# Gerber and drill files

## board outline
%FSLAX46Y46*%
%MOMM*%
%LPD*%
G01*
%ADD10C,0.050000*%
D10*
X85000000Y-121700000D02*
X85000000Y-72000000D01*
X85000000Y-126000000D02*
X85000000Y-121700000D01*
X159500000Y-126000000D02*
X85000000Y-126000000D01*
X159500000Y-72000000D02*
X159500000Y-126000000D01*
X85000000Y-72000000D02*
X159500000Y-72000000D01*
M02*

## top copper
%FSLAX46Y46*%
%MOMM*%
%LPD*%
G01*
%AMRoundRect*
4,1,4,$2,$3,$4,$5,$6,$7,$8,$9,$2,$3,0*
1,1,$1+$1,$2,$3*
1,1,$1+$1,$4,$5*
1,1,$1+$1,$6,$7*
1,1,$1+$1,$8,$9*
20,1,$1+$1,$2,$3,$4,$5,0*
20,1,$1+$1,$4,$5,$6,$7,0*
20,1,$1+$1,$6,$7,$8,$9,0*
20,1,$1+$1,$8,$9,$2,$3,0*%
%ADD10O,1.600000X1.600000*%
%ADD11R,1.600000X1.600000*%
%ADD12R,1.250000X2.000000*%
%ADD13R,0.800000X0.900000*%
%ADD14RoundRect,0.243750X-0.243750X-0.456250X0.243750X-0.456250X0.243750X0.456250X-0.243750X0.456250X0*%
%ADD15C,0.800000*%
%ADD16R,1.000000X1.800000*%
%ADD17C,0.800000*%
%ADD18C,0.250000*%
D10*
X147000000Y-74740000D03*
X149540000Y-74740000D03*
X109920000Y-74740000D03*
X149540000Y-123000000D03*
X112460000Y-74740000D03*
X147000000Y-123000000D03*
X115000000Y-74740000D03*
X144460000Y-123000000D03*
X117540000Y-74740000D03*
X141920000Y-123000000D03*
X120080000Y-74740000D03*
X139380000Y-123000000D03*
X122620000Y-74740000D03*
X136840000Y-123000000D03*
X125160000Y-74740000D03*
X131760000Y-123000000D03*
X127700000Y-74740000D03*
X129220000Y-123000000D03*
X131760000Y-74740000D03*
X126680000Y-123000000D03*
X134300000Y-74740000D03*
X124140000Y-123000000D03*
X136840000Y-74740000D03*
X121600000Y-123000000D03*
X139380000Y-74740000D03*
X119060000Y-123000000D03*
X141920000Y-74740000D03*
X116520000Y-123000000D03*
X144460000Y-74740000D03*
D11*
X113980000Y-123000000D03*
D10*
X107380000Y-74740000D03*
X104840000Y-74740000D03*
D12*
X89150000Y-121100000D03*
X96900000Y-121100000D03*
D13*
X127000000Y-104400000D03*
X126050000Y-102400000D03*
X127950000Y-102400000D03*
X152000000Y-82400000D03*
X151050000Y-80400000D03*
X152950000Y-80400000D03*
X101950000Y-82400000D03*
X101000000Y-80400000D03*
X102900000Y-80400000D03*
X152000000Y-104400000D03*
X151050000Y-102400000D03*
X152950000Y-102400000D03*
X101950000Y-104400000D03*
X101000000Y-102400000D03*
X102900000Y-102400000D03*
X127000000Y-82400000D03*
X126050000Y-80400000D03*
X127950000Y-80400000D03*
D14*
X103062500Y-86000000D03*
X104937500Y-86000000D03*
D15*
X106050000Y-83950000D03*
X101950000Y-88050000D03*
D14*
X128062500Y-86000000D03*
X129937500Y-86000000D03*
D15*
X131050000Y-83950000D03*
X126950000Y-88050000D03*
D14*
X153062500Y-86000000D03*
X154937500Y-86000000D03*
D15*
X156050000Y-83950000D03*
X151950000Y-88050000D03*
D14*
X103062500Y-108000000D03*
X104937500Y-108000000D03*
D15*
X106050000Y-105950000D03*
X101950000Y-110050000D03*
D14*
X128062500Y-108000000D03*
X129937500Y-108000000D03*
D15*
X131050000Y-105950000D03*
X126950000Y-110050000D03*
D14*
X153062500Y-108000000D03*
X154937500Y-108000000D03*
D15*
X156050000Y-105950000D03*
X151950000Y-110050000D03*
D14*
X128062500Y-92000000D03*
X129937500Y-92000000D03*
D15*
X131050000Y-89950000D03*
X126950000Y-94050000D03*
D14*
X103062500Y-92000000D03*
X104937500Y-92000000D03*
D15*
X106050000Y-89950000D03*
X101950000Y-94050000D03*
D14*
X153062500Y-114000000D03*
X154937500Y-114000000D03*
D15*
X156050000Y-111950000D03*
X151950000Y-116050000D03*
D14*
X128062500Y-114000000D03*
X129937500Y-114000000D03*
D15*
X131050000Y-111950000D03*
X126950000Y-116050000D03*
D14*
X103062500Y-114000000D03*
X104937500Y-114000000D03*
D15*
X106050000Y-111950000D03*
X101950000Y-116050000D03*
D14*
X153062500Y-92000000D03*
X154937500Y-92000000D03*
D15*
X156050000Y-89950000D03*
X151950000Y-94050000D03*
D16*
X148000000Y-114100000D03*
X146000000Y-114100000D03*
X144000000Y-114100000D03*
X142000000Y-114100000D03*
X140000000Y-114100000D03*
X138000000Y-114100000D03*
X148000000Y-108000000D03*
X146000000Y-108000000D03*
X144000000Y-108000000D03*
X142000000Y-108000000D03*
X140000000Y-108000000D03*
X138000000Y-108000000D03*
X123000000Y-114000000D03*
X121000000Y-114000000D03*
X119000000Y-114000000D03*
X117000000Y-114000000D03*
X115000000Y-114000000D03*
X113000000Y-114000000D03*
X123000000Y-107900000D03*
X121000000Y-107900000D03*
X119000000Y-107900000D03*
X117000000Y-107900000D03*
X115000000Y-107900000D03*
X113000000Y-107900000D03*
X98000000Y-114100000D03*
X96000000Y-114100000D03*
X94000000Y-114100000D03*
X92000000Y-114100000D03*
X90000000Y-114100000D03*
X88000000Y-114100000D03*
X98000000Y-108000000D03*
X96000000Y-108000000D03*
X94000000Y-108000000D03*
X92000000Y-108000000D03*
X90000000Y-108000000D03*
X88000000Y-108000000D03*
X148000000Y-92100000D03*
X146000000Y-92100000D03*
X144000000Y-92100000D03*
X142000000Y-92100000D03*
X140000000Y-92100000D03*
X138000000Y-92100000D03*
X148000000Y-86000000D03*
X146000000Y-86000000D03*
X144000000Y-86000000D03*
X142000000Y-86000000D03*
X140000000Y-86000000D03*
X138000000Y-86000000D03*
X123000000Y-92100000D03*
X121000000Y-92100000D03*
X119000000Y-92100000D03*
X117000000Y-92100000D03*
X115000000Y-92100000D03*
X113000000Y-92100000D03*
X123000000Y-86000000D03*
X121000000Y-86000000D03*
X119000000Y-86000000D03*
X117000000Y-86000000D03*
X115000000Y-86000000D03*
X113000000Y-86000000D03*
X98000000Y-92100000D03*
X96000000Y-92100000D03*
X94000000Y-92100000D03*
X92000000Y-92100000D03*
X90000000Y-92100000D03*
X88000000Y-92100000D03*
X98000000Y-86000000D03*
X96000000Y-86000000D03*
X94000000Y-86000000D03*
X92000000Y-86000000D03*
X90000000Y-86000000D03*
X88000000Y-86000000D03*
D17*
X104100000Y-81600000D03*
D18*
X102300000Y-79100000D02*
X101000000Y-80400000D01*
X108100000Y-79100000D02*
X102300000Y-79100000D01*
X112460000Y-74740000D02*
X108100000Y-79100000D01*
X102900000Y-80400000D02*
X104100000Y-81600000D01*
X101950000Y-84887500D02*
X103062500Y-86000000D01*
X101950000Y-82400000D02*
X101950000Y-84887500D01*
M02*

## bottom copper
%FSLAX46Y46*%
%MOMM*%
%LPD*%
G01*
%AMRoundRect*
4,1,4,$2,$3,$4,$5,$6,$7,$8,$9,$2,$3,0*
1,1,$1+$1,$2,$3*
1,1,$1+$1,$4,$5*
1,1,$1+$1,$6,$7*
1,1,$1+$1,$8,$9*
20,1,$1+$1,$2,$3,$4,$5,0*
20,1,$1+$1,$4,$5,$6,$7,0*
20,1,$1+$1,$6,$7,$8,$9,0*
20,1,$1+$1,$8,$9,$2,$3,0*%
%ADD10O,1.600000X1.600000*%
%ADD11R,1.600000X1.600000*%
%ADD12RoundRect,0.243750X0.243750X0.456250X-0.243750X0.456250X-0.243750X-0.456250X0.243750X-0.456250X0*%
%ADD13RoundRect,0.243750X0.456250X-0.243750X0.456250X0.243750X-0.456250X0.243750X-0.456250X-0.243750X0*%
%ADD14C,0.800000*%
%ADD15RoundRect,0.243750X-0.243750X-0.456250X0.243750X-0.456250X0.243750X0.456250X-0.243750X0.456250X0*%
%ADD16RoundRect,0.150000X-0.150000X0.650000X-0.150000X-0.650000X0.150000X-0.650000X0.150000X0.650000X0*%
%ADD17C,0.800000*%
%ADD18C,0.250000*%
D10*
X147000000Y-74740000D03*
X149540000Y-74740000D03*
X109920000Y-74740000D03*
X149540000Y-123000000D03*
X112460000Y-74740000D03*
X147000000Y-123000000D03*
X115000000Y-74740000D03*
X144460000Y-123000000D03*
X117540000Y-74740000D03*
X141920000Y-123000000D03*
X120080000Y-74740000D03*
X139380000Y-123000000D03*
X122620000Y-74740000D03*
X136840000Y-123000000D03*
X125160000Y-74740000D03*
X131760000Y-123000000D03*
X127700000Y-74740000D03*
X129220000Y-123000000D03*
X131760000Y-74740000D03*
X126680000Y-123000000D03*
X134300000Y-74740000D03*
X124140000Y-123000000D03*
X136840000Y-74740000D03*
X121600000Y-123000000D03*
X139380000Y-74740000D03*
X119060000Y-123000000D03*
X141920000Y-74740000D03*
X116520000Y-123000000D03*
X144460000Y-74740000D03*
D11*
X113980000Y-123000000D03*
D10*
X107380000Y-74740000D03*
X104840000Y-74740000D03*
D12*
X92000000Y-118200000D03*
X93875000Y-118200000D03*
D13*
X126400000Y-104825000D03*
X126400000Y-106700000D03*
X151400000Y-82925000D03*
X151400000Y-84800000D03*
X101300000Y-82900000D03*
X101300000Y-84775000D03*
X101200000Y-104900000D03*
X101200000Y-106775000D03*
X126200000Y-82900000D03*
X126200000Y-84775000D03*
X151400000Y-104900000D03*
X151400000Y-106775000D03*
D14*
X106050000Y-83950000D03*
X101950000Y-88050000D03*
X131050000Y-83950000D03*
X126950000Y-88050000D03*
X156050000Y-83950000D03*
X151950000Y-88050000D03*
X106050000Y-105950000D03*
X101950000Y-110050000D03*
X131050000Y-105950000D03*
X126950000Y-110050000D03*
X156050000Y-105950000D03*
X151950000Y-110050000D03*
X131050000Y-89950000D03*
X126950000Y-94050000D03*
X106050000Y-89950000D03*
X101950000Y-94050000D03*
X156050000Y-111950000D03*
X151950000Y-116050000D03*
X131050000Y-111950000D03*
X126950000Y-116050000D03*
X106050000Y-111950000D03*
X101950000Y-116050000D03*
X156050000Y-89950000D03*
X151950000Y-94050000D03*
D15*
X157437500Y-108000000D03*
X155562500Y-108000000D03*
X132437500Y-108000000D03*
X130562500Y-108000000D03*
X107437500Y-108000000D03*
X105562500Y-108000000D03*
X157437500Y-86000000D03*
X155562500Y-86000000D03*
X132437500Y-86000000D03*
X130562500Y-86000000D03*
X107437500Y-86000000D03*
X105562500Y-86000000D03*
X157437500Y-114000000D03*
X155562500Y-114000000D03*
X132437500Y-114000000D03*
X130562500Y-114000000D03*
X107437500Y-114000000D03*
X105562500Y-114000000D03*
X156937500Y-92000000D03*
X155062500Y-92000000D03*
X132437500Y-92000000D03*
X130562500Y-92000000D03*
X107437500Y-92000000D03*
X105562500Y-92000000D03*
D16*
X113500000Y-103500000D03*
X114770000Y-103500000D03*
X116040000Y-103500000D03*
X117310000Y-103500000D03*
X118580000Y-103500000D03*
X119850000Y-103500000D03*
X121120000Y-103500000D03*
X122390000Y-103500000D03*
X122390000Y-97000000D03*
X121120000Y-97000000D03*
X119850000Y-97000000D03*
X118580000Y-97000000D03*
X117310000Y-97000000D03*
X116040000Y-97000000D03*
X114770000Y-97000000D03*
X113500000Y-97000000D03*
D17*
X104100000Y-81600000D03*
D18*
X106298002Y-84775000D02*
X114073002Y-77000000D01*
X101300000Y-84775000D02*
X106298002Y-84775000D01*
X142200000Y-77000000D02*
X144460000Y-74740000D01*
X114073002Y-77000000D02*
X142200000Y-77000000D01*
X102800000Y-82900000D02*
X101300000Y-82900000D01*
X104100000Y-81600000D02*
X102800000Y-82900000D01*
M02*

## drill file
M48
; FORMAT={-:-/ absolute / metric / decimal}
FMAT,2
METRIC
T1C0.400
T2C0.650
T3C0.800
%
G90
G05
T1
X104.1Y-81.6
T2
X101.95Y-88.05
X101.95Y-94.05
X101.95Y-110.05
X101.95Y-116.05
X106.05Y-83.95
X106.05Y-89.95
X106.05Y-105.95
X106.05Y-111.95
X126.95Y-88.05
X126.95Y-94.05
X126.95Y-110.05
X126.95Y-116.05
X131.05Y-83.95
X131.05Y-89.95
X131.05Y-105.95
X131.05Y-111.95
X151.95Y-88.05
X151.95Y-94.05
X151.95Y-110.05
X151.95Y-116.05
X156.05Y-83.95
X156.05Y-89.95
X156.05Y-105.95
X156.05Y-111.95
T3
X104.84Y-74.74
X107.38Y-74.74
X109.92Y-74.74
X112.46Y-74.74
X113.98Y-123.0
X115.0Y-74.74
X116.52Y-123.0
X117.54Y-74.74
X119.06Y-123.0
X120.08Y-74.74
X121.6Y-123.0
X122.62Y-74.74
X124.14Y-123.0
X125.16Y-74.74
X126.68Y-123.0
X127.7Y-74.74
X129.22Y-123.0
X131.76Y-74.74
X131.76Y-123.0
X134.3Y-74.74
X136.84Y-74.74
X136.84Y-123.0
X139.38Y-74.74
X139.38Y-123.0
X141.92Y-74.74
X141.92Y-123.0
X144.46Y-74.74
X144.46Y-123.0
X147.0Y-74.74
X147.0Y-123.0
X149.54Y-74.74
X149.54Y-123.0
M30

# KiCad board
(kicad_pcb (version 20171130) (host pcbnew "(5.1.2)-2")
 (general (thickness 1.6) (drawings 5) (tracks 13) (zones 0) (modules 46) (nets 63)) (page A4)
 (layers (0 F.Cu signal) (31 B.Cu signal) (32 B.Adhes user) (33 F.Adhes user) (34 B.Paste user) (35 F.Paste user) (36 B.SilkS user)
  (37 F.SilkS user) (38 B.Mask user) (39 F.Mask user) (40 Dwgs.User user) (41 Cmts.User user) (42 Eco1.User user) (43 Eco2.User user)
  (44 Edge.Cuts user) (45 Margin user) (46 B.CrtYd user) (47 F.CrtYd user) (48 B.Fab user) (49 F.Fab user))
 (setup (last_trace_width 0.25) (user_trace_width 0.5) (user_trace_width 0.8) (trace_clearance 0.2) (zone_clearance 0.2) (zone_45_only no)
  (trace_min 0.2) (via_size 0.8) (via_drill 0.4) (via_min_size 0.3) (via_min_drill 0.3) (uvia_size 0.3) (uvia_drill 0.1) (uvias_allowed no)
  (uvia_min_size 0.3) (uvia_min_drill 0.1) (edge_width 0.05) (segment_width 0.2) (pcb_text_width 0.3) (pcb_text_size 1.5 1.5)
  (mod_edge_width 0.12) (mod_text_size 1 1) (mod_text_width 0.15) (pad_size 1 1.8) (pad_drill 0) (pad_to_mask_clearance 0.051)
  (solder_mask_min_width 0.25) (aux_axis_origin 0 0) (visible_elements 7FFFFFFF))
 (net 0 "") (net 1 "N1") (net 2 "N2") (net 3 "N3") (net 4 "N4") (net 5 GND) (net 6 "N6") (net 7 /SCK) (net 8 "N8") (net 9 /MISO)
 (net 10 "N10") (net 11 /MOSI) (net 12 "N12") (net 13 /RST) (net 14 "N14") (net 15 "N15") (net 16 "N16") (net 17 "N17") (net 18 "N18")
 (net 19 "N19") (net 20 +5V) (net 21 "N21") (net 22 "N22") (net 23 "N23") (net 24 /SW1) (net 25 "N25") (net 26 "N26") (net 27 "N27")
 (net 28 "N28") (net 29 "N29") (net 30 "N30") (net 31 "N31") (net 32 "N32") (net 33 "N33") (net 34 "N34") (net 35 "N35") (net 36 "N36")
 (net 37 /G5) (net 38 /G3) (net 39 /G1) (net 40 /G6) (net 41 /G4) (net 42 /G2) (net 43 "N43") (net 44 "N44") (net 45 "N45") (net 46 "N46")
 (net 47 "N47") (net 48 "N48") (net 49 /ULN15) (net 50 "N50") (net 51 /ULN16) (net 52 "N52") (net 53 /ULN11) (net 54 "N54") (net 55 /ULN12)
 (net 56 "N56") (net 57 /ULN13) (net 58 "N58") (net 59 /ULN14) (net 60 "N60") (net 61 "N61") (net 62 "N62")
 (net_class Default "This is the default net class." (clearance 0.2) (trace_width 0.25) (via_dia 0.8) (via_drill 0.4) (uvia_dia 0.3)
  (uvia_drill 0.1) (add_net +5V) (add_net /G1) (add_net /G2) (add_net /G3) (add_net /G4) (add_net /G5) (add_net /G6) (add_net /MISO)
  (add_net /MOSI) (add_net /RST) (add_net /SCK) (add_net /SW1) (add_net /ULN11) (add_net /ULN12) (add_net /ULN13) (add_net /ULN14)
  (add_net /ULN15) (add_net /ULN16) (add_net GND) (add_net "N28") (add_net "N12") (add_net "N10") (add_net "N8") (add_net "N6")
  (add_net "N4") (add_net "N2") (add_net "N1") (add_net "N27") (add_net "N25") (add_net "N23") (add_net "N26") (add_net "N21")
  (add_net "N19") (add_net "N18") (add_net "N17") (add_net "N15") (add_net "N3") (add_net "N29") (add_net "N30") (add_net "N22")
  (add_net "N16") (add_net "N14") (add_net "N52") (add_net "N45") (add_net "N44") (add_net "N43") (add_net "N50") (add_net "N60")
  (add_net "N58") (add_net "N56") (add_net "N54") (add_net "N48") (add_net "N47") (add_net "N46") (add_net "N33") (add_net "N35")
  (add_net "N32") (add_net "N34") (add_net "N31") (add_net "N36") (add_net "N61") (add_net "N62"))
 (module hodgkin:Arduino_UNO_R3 (layer B.Cu) (at 113.98 123)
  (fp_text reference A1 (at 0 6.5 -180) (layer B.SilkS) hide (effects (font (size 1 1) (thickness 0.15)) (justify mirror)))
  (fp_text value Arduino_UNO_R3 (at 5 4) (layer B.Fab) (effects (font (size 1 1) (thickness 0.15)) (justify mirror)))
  (pad 16 thru_hole oval (at 33.02 -48.26 270) (size 1.6 1.6) (drill 0.8) (layers *.Cu *.Mask) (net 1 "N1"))
  (pad 15 thru_hole oval (at 35.56 -48.26 270) (size 1.6 1.6) (drill 0.8) (layers *.Cu *.Mask) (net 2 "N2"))
  (pad 30 thru_hole oval (at -4.06 -48.26 270) (size 1.6 1.6) (drill 0.8) (layers *.Cu *.Mask) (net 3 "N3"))
  (pad 14 thru_hole oval (at 35.56 0 270) (size 1.6 1.6) (drill 0.8) (layers *.Cu *.Mask) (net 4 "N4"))
  (pad 29 thru_hole oval (at -1.52 -48.26 270) (size 1.6 1.6) (drill 0.8) (layers *.Cu *.Mask) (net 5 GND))
  (pad 13 thru_hole oval (at 33.02 0 270) (size 1.6 1.6) (drill 0.8) (layers *.Cu *.Mask) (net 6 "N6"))
  (pad 28 thru_hole oval (at 1.02 -48.26 270) (size 1.6 1.6) (drill 0.8) (layers *.Cu *.Mask) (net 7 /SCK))
  (pad 12 thru_hole oval (at 30.48 0 270) (size 1.6 1.6) (drill 0.8) (layers *.Cu *.Mask) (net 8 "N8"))
  (pad 27 thru_hole oval (at 3.56 -48.26 270) (size 1.6 1.6) (drill 0.8) (layers *.Cu *.Mask) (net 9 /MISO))
  (pad 11 thru_hole oval (at 27.94 0 270) (size 1.6 1.6) (drill 0.8) (layers *.Cu *.Mask) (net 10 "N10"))
  (pad 26 thru_hole oval (at 6.1 -48.26 270) (size 1.6 1.6) (drill 0.8) (layers *.Cu *.Mask) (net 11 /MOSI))
  (pad 10 thru_hole oval (at 25.4 0 270) (size 1.6 1.6) (drill 0.8) (layers *.Cu *.Mask) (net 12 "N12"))
  (pad 25 thru_hole oval (at 8.64 -48.26 270) (size 1.6 1.6) (drill 0.8) (layers *.Cu *.Mask) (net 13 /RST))
  (pad 9 thru_hole oval (at 22.86 0 270) (size 1.6 1.6) (drill 0.8) (layers *.Cu *.Mask) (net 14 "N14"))
  (pad 24 thru_hole oval (at 11.18 -48.26 270) (size 1.6 1.6) (drill 0.8) (layers *.Cu *.Mask) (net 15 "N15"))
  (pad 8 thru_hole oval (at 17.78 0 270) (size 1.6 1.6) (drill 0.8) (layers *.Cu *.Mask) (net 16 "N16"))
  (pad 23 thru_hole oval (at 13.72 -48.26 270) (size 1.6 1.6) (drill 0.8) (layers *.Cu *.Mask) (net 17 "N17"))
  (pad 7 thru_hole oval (at 15.24 0 270) (size 1.6 1.6) (drill 0.8) (layers *.Cu *.Mask) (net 5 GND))
  (pad 22 thru_hole oval (at 17.78 -48.26 270) (size 1.6 1.6) (drill 0.8) (layers *.Cu *.Mask) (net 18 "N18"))
  (pad 6 thru_hole oval (at 12.7 0 270) (size 1.6 1.6) (drill 0.8) (layers *.Cu *.Mask) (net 5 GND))
  (pad 21 thru_hole oval (at 20.32 -48.26 270) (size 1.6 1.6) (drill 0.8) (layers *.Cu *.Mask) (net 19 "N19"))
  (pad 5 thru_hole oval (at 10.16 0 270) (size 1.6 1.6) (drill 0.8) (layers *.Cu *.Mask) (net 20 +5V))
  (pad 20 thru_hole oval (at 22.86 -48.26 270) (size 1.6 1.6) (drill 0.8) (layers *.Cu *.Mask) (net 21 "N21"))
  (pad 4 thru_hole oval (at 7.62 0 270) (size 1.6 1.6) (drill 0.8) (layers *.Cu *.Mask) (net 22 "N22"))
  (pad 19 thru_hole oval (at 25.4 -48.26 270) (size 1.6 1.6) (drill 0.8) (layers *.Cu *.Mask) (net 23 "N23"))
  (pad 3 thru_hole oval (at 5.08 0 270) (size 1.6 1.6) (drill 0.8) (layers *.Cu *.Mask) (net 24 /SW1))
  (pad 18 thru_hole oval (at 27.94 -48.26 270) (size 1.6 1.6) (drill 0.8) (layers *.Cu *.Mask) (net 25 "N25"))
  (pad 2 thru_hole oval (at 2.54 0 270) (size 1.6 1.6) (drill 0.8) (layers *.Cu *.Mask) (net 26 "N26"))
  (pad 17 thru_hole oval (at 30.48 -48.26 270) (size 1.6 1.6) (drill 0.8) (layers *.Cu *.Mask) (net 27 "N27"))
  (pad 1 thru_hole rect (at 0 0 270) (size 1.6 1.6) (drill 0.8) (layers *.Cu *.Mask) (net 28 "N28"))
  (pad 31 thru_hole oval (at -6.6 -48.26 270) (size 1.6 1.6) (drill 0.8) (layers *.Cu *.Mask) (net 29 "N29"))
  (pad 32 thru_hole oval (at -9.14 -48.26 270) (size 1.6 1.6) (drill 0.8) (layers *.Cu *.Mask) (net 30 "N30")))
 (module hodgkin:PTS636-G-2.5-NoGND (layer F.Cu) (at 96.9 121.1 180)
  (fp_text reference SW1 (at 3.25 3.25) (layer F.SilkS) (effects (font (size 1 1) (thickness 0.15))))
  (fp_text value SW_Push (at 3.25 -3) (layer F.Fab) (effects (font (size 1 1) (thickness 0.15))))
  (pad 2 smd rect (at 7.75 0 180) (size 1.25 2) (layers F.Cu F.Paste F.Mask) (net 24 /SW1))
  (pad 1 smd rect (at 0 0 180) (size 1.25 2) (layers F.Cu F.Paste F.Mask) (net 5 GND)))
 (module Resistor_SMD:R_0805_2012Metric (layer B.Cu) (at 92.9375 118.2 180)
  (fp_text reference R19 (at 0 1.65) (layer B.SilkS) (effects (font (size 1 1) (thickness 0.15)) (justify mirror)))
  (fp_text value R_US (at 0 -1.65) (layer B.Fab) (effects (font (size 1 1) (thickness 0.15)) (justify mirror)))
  (pad 2 smd roundrect (at 0.9375 0 180) (size 0.975 1.4) (layers B.Cu B.Paste B.Mask) (roundrect_rratio 0.25) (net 24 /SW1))
  (pad 1 smd roundrect (at -0.9375 0 180) (size 0.975 1.4) (layers B.Cu B.Paste B.Mask) (roundrect_rratio 0.25) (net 20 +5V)))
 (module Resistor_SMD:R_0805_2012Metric (layer B.Cu) (at 126.4 105.7625 90)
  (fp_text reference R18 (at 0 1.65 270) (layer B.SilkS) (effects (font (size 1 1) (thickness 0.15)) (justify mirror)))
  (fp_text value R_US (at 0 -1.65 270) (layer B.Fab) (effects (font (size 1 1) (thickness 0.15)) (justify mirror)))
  (pad 2 smd roundrect (at 0.9375 0 90) (size 0.975 1.4) (layers B.Cu B.Paste B.Mask) (roundrect_rratio 0.25) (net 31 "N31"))
  (pad 1 smd roundrect (at -0.9375 0 90) (size 0.975 1.4) (layers B.Cu B.Paste B.Mask) (roundrect_rratio 0.25) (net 6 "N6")))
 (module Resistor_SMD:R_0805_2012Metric (layer B.Cu) (at 151.4 83.8625 90)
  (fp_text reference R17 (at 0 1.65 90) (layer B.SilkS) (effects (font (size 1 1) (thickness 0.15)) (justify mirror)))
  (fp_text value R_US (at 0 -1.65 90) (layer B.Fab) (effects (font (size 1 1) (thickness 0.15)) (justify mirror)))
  (pad 2 smd roundrect (at 0.9375 0 90) (size 0.975 1.4) (layers B.Cu B.Paste B.Mask) (roundrect_rratio 0.25) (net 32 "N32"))
  (pad 1 smd roundrect (at -0.9375 0 90) (size 0.975 1.4) (layers B.Cu B.Paste B.Mask) (roundrect_rratio 0.25) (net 2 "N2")))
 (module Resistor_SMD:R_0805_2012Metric (layer B.Cu) (at 101.3 83.8375 90)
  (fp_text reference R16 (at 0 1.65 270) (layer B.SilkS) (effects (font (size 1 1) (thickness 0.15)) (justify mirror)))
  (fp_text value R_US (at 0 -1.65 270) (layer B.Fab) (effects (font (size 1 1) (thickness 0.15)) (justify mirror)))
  (pad 2 smd roundrect (at 0.9375 0 90) (size 0.975 1.4) (layers B.Cu B.Paste B.Mask) (roundrect_rratio 0.25) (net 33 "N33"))
  (pad 1 smd roundrect (at -0.9375 0 90) (size 0.975 1.4) (layers B.Cu B.Paste B.Mask) (roundrect_rratio 0.25) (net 27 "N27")))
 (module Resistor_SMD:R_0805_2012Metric (layer B.Cu) (at 101.2 105.8375 90)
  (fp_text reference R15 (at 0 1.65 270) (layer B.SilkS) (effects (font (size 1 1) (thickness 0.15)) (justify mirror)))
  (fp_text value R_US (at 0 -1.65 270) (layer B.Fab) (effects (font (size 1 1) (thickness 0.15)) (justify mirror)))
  (pad 2 smd roundrect (at 0.9375 0 90) (size 0.975 1.4) (layers B.Cu B.Paste B.Mask) (roundrect_rratio 0.25) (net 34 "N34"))
  (pad 1 smd roundrect (at -0.9375 0 90) (size 0.975 1.4) (layers B.Cu B.Paste B.Mask) (roundrect_rratio 0.25) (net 8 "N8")))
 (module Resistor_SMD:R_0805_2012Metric (layer B.Cu) (at 126.2 83.8375 90)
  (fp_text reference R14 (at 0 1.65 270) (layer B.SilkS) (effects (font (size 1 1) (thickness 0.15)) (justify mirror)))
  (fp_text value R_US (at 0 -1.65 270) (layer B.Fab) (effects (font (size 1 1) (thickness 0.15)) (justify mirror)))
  (pad 2 smd roundrect (at 0.9375 0 90) (size 0.975 1.4) (layers B.Cu B.Paste B.Mask) (roundrect_rratio 0.25) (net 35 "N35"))
  (pad 1 smd roundrect (at -0.9375 0 90) (size 0.975 1.4) (layers B.Cu B.Paste B.Mask) (roundrect_rratio 0.25) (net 1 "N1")))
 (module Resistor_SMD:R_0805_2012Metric (layer B.Cu) (at 151.4 105.8375 90)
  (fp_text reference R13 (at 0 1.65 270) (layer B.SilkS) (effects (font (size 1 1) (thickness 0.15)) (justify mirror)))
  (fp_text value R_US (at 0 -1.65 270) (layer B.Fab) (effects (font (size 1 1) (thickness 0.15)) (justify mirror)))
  (pad 2 smd roundrect (at 0.9375 0 90) (size 0.975 1.4) (layers B.Cu B.Paste B.Mask) (roundrect_rratio 0.25) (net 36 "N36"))
  (pad 1 smd roundrect (at -0.9375 0 90) (size 0.975 1.4) (layers B.Cu B.Paste B.Mask) (roundrect_rratio 0.25) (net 4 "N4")))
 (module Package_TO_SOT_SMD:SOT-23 (layer F.Cu) (at 127 103.4 270)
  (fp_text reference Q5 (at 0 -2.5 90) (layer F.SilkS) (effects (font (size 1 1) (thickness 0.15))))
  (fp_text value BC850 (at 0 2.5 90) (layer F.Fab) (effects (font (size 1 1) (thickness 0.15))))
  (pad 3 smd rect (at 1 0 270) (size 0.9 0.8) (layers F.Cu F.Paste F.Mask) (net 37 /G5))
  (pad 2 smd rect (at -1 0.95 270) (size 0.9 0.8) (layers F.Cu F.Paste F.Mask) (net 5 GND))
  (pad 1 smd rect (at -1 -0.95 270) (size 0.9 0.8) (layers F.Cu F.Paste F.Mask) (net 31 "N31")))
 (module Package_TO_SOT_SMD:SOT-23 (layer F.Cu) (at 152 81.4 270)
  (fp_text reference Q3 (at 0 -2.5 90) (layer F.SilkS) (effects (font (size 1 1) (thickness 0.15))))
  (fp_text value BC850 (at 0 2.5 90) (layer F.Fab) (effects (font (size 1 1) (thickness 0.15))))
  (pad 3 smd rect (at 1 0 270) (size 0.9 0.8) (layers F.Cu F.Paste F.Mask) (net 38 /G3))
  (pad 2 smd rect (at -1 0.95 270) (size 0.9 0.8) (layers F.Cu F.Paste F.Mask) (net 5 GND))
  (pad 1 smd rect (at -1 -0.95 270) (size 0.9 0.8) (layers F.Cu F.Paste F.Mask) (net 32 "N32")))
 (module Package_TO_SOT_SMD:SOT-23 (layer F.Cu) (at 101.95 81.4 270)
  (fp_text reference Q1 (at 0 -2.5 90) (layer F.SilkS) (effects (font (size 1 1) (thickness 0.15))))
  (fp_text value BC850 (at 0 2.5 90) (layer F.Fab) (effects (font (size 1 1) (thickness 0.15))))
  (pad 3 smd rect (at 1 0 270) (size 0.9 0.8) (layers F.Cu F.Paste F.Mask) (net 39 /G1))
  (pad 2 smd rect (at -1 0.95 270) (size 0.9 0.8) (layers F.Cu F.Paste F.Mask) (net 5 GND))
  (pad 1 smd rect (at -1 -0.95 270) (size 0.9 0.8) (layers F.Cu F.Paste F.Mask) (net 33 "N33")))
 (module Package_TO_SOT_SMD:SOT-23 (layer F.Cu) (at 152 103.4 270)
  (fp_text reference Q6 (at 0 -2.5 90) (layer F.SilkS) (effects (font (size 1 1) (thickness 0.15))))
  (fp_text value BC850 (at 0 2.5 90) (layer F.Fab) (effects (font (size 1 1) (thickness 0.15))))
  (pad 3 smd rect (at 1 0 270) (size 0.9 0.8) (layers F.Cu F.Paste F.Mask) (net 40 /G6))
  (pad 2 smd rect (at -1 0.95 270) (size 0.9 0.8) (layers F.Cu F.Paste F.Mask) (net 5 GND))
  (pad 1 smd rect (at -1 -0.95 270) (size 0.9 0.8) (layers F.Cu F.Paste F.Mask) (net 36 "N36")))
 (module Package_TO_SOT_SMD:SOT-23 (layer F.Cu) (at 101.95 103.4 270)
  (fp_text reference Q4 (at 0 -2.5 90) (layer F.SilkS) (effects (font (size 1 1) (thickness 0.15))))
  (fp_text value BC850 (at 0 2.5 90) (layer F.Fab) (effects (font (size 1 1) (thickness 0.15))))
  (pad 3 smd rect (at 1 0 270) (size 0.9 0.8) (layers F.Cu F.Paste F.Mask) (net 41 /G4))
  (pad 2 smd rect (at -1 0.95 270) (size 0.9 0.8) (layers F.Cu F.Paste F.Mask) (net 5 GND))
  (pad 1 smd rect (at -1 -0.95 270) (size 0.9 0.8) (layers F.Cu F.Paste F.Mask) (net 34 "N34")))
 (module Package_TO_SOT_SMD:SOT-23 (layer F.Cu) (at 127 81.4 270)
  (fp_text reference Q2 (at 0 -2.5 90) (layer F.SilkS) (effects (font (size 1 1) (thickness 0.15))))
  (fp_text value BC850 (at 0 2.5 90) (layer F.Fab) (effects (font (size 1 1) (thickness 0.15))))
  (pad 3 smd rect (at 1 0 270) (size 0.9 0.8) (layers F.Cu F.Paste F.Mask) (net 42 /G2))
  (pad 2 smd rect (at -1 0.95 270) (size 0.9 0.8) (layers F.Cu F.Paste F.Mask) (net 5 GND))
  (pad 1 smd rect (at -1 -0.95 270) (size 0.9 0.8) (layers F.Cu F.Paste F.Mask) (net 35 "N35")))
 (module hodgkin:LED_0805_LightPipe (layer F.Cu) (at 104 86)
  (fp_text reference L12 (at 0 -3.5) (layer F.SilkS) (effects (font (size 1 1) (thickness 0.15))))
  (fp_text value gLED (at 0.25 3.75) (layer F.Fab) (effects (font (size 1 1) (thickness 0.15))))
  (pad 1 smd roundrect (at -0.9375 0) (size 0.975 1.4) (layers F.Cu F.Paste F.Mask) (roundrect_rratio 0.25) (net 39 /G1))
  (pad 2 smd roundrect (at 0.9375 0) (size 0.975 1.4) (layers F.Cu F.Paste F.Mask) (roundrect_rratio 0.25) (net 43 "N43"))
  (pad "" thru_hole circle (at 2.05 -2.05) (size 0.8 0.8) (drill 0.65) (layers *.Cu *.Mask))
  (pad "" thru_hole circle (at -2.05 2.05) (size 0.8 0.8) (drill 0.65) (layers *.Cu *.Mask)))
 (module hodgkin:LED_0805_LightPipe (layer F.Cu) (at 129 86)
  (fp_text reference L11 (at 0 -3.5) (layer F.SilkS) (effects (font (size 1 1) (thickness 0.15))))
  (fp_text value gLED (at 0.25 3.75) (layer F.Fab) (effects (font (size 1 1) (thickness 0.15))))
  (pad 1 smd roundrect (at -0.9375 0) (size 0.975 1.4) (layers F.Cu F.Paste F.Mask) (roundrect_rratio 0.25) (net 42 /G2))
  (pad 2 smd roundrect (at 0.9375 0) (size 0.975 1.4) (layers F.Cu F.Paste F.Mask) (roundrect_rratio 0.25) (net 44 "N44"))
  (pad "" thru_hole circle (at 2.05 -2.05) (size 0.8 0.8) (drill 0.65) (layers *.Cu *.Mask))
  (pad "" thru_hole circle (at -2.05 2.05) (size 0.8 0.8) (drill 0.65) (layers *.Cu *.Mask)))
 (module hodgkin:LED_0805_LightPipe (layer F.Cu) (at 154 86)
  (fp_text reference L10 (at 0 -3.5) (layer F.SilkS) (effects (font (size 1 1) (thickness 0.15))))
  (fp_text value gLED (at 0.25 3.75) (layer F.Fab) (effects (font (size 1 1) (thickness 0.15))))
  (pad 1 smd roundrect (at -0.9375 0) (size 0.975 1.4) (layers F.Cu F.Paste F.Mask) (roundrect_rratio 0.25) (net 38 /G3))
  (pad 2 smd roundrect (at 0.9375 0) (size 0.975 1.4) (layers F.Cu F.Paste F.Mask) (roundrect_rratio 0.25) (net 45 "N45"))
  (pad "" thru_hole circle (at 2.05 -2.05) (size 0.8 0.8) (drill 0.65) (layers *.Cu *.Mask))
  (pad "" thru_hole circle (at -2.05 2.05) (size 0.8 0.8) (drill 0.65) (layers *.Cu *.Mask)))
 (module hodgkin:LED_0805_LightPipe (layer F.Cu) (at 104 108)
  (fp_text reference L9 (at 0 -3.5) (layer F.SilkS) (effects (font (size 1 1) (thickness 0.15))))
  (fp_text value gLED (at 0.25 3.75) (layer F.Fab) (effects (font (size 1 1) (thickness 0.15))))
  (pad 1 smd roundrect (at -0.9375 0) (size 0.975 1.4) (layers F.Cu F.Paste F.Mask) (roundrect_rratio 0.25) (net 41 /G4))
  (pad 2 smd roundrect (at 0.9375 0) (size 0.975 1.4) (layers F.Cu F.Paste F.Mask) (roundrect_rratio 0.25) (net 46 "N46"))
  (pad "" thru_hole circle (at 2.05 -2.05) (size 0.8 0.8) (drill 0.65) (layers *.Cu *.Mask))
  (pad "" thru_hole circle (at -2.05 2.05) (size 0.8 0.8) (drill 0.65) (layers *.Cu *.Mask)))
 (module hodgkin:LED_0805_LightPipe (layer F.Cu) (at 129 108)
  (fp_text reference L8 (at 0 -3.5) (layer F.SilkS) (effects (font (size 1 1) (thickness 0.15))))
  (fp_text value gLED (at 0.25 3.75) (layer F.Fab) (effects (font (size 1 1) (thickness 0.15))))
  (pad 1 smd roundrect (at -0.9375 0) (size 0.975 1.4) (layers F.Cu F.Paste F.Mask) (roundrect_rratio 0.25) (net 37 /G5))
  (pad 2 smd roundrect (at 0.9375 0) (size 0.975 1.4) (layers F.Cu F.Paste F.Mask) (roundrect_rratio 0.25) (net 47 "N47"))
  (pad "" thru_hole circle (at 2.05 -2.05) (size 0.8 0.8) (drill 0.65) (layers *.Cu *.Mask))
  (pad "" thru_hole circle (at -2.05 2.05) (size 0.8 0.8) (drill 0.65) (layers *.Cu *.Mask)))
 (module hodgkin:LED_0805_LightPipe (layer F.Cu) (at 154 108)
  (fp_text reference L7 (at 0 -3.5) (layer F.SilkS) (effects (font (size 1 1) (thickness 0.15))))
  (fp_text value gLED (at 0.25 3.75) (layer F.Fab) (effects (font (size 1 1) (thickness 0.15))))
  (pad 1 smd roundrect (at -0.9375 0) (size 0.975 1.4) (layers F.Cu F.Paste F.Mask) (roundrect_rratio 0.25) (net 40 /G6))
  (pad 2 smd roundrect (at 0.9375 0) (size 0.975 1.4) (layers F.Cu F.Paste F.Mask) (roundrect_rratio 0.25) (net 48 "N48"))
  (pad "" thru_hole circle (at 2.05 -2.05) (size 0.8 0.8) (drill 0.65) (layers *.Cu *.Mask))
  (pad "" thru_hole circle (at -2.05 2.05) (size 0.8 0.8) (drill 0.65) (layers *.Cu *.Mask)))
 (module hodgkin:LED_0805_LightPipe (layer F.Cu) (at 129 92)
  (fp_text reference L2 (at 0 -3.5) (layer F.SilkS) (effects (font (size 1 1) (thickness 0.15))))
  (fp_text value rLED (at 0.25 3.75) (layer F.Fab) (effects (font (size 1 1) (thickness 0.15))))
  (pad 1 smd roundrect (at -0.9375 0) (size 0.975 1.4) (layers F.Cu F.Paste F.Mask) (roundrect_rratio 0.25) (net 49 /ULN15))
  (pad 2 smd roundrect (at 0.9375 0) (size 0.975 1.4) (layers F.Cu F.Paste F.Mask) (roundrect_rratio 0.25) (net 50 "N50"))
  (pad "" thru_hole circle (at 2.05 -2.05) (size 0.8 0.8) (drill 0.65) (layers *.Cu *.Mask))
  (pad "" thru_hole circle (at -2.05 2.05) (size 0.8 0.8) (drill 0.65) (layers *.Cu *.Mask)))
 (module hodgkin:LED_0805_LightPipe (layer F.Cu) (at 104 92)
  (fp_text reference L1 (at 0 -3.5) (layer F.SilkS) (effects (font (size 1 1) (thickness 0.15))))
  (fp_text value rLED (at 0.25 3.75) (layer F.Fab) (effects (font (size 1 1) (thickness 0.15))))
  (pad 1 smd roundrect (at -0.9375 0) (size 0.975 1.4) (layers F.Cu F.Paste F.Mask) (roundrect_rratio 0.25) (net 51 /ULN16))
  (pad 2 smd roundrect (at 0.9375 0) (size 0.975 1.4) (layers F.Cu F.Paste F.Mask) (roundrect_rratio 0.25) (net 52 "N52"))
  (pad "" thru_hole circle (at 2.05 -2.05) (size 0.8 0.8) (drill 0.65) (layers *.Cu *.Mask))
  (pad "" thru_hole circle (at -2.05 2.05) (size 0.8 0.8) (drill 0.65) (layers *.Cu *.Mask)))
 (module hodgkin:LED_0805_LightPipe (layer F.Cu) (at 154 114)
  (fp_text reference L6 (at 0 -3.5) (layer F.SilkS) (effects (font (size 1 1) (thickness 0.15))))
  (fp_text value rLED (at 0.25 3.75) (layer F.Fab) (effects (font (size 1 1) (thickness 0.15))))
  (pad 1 smd roundrect (at -0.9375 0) (size 0.975 1.4) (layers F.Cu F.Paste F.Mask) (roundrect_rratio 0.25) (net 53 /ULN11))
  (pad 2 smd roundrect (at 0.9375 0) (size 0.975 1.4) (layers F.Cu F.Paste F.Mask) (roundrect_rratio 0.25) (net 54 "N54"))
  (pad "" thru_hole circle (at 2.05 -2.05) (size 0.8 0.8) (drill 0.65) (layers *.Cu *.Mask))
  (pad "" thru_hole circle (at -2.05 2.05) (size 0.8 0.8) (drill 0.65) (layers *.Cu *.Mask)))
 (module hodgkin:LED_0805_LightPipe (layer F.Cu) (at 129 114)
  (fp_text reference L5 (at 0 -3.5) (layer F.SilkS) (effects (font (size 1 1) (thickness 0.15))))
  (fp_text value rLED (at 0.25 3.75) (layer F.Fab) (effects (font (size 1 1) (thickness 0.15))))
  (pad 1 smd roundrect (at -0.9375 0) (size 0.975 1.4) (layers F.Cu F.Paste F.Mask) (roundrect_rratio 0.25) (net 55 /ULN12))
  (pad 2 smd roundrect (at 0.9375 0) (size 0.975 1.4) (layers F.Cu F.Paste F.Mask) (roundrect_rratio 0.25) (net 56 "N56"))
  (pad "" thru_hole circle (at 2.05 -2.05) (size 0.8 0.8) (drill 0.65) (layers *.Cu *.Mask))
  (pad "" thru_hole circle (at -2.05 2.05) (size 0.8 0.8) (drill 0.65) (layers *.Cu *.Mask)))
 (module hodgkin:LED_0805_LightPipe (layer F.Cu) (at 104 114)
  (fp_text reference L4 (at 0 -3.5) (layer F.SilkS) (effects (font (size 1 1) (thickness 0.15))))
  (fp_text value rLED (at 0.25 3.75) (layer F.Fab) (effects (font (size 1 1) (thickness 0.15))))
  (pad 1 smd roundrect (at -0.9375 0) (size 0.975 1.4) (layers F.Cu F.Paste F.Mask) (roundrect_rratio 0.25) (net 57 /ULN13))
  (pad 2 smd roundrect (at 0.9375 0) (size 0.975 1.4) (layers F.Cu F.Paste F.Mask) (roundrect_rratio 0.25) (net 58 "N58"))
  (pad "" thru_hole circle (at 2.05 -2.05) (size 0.8 0.8) (drill 0.65) (layers *.Cu *.Mask))
  (pad "" thru_hole circle (at -2.05 2.05) (size 0.8 0.8) (drill 0.65) (layers *.Cu *.Mask)))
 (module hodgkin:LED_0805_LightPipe (layer F.Cu) (at 154 92)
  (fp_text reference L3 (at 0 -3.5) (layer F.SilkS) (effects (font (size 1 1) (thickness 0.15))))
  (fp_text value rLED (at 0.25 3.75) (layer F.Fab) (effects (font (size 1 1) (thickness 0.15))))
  (pad 1 smd roundrect (at -0.9375 0) (size 0.975 1.4) (layers F.Cu F.Paste F.Mask) (roundrect_rratio 0.25) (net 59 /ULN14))
  (pad 2 smd roundrect (at 0.9375 0) (size 0.975 1.4) (layers F.Cu F.Paste F.Mask) (roundrect_rratio 0.25) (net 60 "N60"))
  (pad "" thru_hole circle (at 2.05 -2.05) (size 0.8 0.8) (drill 0.65) (layers *.Cu *.Mask))
  (pad "" thru_hole circle (at -2.05 2.05) (size 0.8 0.8) (drill 0.65) (layers *.Cu *.Mask)))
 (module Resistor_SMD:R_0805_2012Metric (layer B.Cu) (at 156.5 108)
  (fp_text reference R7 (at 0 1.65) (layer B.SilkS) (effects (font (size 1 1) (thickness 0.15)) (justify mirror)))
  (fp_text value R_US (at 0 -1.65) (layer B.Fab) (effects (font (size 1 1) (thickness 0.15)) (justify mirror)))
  (pad 2 smd roundrect (at 0.9375 0) (size 0.975 1.4) (layers B.Cu B.Paste B.Mask) (roundrect_rratio 0.25) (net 48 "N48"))
  (pad 1 smd roundrect (at -0.9375 0) (size 0.975 1.4) (layers B.Cu B.Paste B.Mask) (roundrect_rratio 0.25) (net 20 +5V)))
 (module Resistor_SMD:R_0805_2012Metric (layer B.Cu) (at 131.5 108)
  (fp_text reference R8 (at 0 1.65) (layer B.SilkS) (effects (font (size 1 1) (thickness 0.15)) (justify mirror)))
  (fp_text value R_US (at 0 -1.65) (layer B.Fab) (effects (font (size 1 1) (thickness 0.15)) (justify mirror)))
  (pad 2 smd roundrect (at 0.9375 0) (size 0.975 1.4) (layers B.Cu B.Paste B.Mask) (roundrect_rratio 0.25) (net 47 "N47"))
  (pad 1 smd roundrect (at -0.9375 0) (size 0.975 1.4) (layers B.Cu B.Paste B.Mask) (roundrect_rratio 0.25) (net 20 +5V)))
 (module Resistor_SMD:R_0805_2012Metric (layer B.Cu) (at 106.5 108)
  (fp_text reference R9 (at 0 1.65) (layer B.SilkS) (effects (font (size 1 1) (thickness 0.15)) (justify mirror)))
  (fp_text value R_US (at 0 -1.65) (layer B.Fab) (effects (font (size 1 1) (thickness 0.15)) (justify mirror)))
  (pad 2 smd roundrect (at 0.9375 0) (size 0.975 1.4) (layers B.Cu B.Paste B.Mask) (roundrect_rratio 0.25) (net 46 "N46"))
  (pad 1 smd roundrect (at -0.9375 0) (size 0.975 1.4) (layers B.Cu B.Paste B.Mask) (roundrect_rratio 0.25) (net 20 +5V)))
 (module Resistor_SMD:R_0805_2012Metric (layer B.Cu) (at 156.5 86)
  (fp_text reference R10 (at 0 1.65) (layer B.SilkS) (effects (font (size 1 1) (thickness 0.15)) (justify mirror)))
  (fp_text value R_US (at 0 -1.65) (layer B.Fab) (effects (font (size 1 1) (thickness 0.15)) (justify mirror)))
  (pad 2 smd roundrect (at 0.9375 0) (size 0.975 1.4) (layers B.Cu B.Paste B.Mask) (roundrect_rratio 0.25) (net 45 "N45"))
  (pad 1 smd roundrect (at -0.9375 0) (size 0.975 1.4) (layers B.Cu B.Paste B.Mask) (roundrect_rratio 0.25) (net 20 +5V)))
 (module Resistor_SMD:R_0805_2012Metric (layer B.Cu) (at 131.5 86)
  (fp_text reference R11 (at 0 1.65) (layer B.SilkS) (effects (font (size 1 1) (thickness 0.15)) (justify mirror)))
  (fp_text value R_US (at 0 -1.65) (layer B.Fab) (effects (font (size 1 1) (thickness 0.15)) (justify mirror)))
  (pad 2 smd roundrect (at 0.9375 0) (size 0.975 1.4) (layers B.Cu B.Paste B.Mask) (roundrect_rratio 0.25) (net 44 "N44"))
  (pad 1 smd roundrect (at -0.9375 0) (size 0.975 1.4) (layers B.Cu B.Paste B.Mask) (roundrect_rratio 0.25) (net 20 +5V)))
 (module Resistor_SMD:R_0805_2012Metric (layer B.Cu) (at 106.5 86)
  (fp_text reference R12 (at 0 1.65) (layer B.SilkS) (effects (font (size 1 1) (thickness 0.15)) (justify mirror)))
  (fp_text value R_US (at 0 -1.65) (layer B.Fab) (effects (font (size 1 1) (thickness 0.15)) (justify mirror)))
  (pad 2 smd roundrect (at 0.9375 0) (size 0.975 1.4) (layers B.Cu B.Paste B.Mask) (roundrect_rratio 0.25) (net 43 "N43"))
  (pad 1 smd roundrect (at -0.9375 0) (size 0.975 1.4) (layers B.Cu B.Paste B.Mask) (roundrect_rratio 0.25) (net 20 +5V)))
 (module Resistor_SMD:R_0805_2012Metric (layer B.Cu) (at 156.5 114)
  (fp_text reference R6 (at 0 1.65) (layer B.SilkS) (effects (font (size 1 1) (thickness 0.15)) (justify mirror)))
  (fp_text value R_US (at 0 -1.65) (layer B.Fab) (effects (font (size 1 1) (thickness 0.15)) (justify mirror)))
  (pad 2 smd roundrect (at 0.9375 0) (size 0.975 1.4) (layers B.Cu B.Paste B.Mask) (roundrect_rratio 0.25) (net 54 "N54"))
  (pad 1 smd roundrect (at -0.9375 0) (size 0.975 1.4) (layers B.Cu B.Paste B.Mask) (roundrect_rratio 0.25) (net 20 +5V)))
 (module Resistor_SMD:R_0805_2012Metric (layer B.Cu) (at 131.5 114)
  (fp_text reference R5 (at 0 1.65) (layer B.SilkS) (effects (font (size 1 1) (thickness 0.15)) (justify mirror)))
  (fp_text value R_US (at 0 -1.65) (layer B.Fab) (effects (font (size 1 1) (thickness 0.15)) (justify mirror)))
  (pad 2 smd roundrect (at 0.9375 0) (size 0.975 1.4) (layers B.Cu B.Paste B.Mask) (roundrect_rratio 0.25) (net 56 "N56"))
  (pad 1 smd roundrect (at -0.9375 0) (size 0.975 1.4) (layers B.Cu B.Paste B.Mask) (roundrect_rratio 0.25) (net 20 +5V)))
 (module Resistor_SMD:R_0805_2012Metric (layer B.Cu) (at 106.5 114)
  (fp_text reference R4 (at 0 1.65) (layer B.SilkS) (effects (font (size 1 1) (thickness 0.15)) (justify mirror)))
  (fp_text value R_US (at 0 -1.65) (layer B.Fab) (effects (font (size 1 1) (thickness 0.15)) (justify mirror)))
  (pad 2 smd roundrect (at 0.9375 0) (size 0.975 1.4) (layers B.Cu B.Paste B.Mask) (roundrect_rratio 0.25) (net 58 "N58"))
  (pad 1 smd roundrect (at -0.9375 0) (size 0.975 1.4) (layers B.Cu B.Paste B.Mask) (roundrect_rratio 0.25) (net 20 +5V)))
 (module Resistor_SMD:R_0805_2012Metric (layer B.Cu) (at 156 92)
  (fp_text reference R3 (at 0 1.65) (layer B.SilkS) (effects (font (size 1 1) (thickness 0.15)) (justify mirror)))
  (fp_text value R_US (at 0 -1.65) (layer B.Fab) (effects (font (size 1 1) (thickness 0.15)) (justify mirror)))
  (pad 2 smd roundrect (at 0.9375 0) (size 0.975 1.4) (layers B.Cu B.Paste B.Mask) (roundrect_rratio 0.25) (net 60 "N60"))
  (pad 1 smd roundrect (at -0.9375 0) (size 0.975 1.4) (layers B.Cu B.Paste B.Mask) (roundrect_rratio 0.25) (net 20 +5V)))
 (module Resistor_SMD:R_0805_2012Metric (layer B.Cu) (at 131.5 92)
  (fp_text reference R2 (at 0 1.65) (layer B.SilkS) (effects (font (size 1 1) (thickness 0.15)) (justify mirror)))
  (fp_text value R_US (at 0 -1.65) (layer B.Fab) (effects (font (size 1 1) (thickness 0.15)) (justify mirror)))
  (pad 2 smd roundrect (at 0.9375 0) (size 0.975 1.4) (layers B.Cu B.Paste B.Mask) (roundrect_rratio 0.25) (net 50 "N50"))
  (pad 1 smd roundrect (at -0.9375 0) (size 0.975 1.4) (layers B.Cu B.Paste B.Mask) (roundrect_rratio 0.25) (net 20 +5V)))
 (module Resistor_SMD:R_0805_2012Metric (layer B.Cu) (at 106.5 92)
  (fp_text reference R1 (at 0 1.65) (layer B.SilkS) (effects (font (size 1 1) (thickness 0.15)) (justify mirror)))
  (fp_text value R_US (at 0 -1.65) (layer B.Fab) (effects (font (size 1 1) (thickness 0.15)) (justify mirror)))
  (pad 2 smd roundrect (at 0.9375 0) (size 0.975 1.4) (layers B.Cu B.Paste B.Mask) (roundrect_rratio 0.25) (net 52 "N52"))
  (pad 1 smd roundrect (at -0.9375 0) (size 0.975 1.4) (layers B.Cu B.Paste B.Mask) (roundrect_rratio 0.25) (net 20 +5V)))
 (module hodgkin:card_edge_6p (layer F.Cu) (at 138 108)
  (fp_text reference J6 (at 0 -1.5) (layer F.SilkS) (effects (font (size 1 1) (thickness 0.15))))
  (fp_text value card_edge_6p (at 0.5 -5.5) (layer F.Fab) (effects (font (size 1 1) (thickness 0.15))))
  (pad 6 smd rect (at 10 6.1) (size 1 1.8) (layers F.Cu F.Paste F.Mask) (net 53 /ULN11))
  (pad 5 smd rect (at 8 6.1) (size 1 1.8) (layers F.Cu F.Paste F.Mask) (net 13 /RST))
  (pad 4 smd rect (at 6 6.1) (size 1 1.8) (layers F.Cu F.Paste F.Mask) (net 11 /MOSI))
  (pad 3 smd rect (at 4 6.1) (size 1 1.8) (layers F.Cu F.Paste F.Mask) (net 9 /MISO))
  (pad 2 smd rect (at 2 6.1) (size 1 1.8) (layers F.Cu F.Paste F.Mask) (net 7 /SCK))
  (pad 1 smd rect (at 0 6.1) (size 1 1.8) (layers F.Cu F.Paste F.Mask) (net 20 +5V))
  (pad 6 smd rect (at 10 0) (size 1 1.8) (layers F.Cu F.Paste F.Mask) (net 53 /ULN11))
  (pad 5 smd rect (at 8 0) (size 1 1.8) (layers F.Cu F.Paste F.Mask) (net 13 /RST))
  (pad 4 smd rect (at 6 0) (size 1 1.8) (layers F.Cu F.Paste F.Mask) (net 11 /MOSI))
  (pad 3 smd rect (at 4 0) (size 1 1.8) (layers F.Cu F.Paste F.Mask) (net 9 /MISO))
  (pad 2 smd rect (at 2 0) (size 1 1.8) (layers F.Cu F.Paste F.Mask) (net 7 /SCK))
  (pad 1 smd rect (at 0 0) (size 1 1.8) (layers F.Cu F.Paste F.Mask) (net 20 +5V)))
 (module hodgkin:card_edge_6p (layer F.Cu) (at 113 107.9)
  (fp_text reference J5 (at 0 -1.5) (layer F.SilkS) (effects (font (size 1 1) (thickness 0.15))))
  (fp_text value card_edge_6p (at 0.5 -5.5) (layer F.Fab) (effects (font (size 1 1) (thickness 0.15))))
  (pad 6 smd rect (at 10 6.1) (size 1 1.8) (layers F.Cu F.Paste F.Mask) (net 55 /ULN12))
  (pad 5 smd rect (at 8 6.1) (size 1 1.8) (layers F.Cu F.Paste F.Mask) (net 13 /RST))
  (pad 4 smd rect (at 6 6.1) (size 1 1.8) (layers F.Cu F.Paste F.Mask) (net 11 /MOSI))
  (pad 3 smd rect (at 4 6.1) (size 1 1.8) (layers F.Cu F.Paste F.Mask) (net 9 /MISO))
  (pad 2 smd rect (at 2 6.1) (size 1 1.8) (layers F.Cu F.Paste F.Mask) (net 7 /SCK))
  (pad 1 smd rect (at 0 6.1) (size 1 1.8) (layers F.Cu F.Paste F.Mask) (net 20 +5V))
  (pad 6 smd rect (at 10 0) (size 1 1.8) (layers F.Cu F.Paste F.Mask) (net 55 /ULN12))
  (pad 5 smd rect (at 8 0) (size 1 1.8) (layers F.Cu F.Paste F.Mask) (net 13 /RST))
  (pad 4 smd rect (at 6 0) (size 1 1.8) (layers F.Cu F.Paste F.Mask) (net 11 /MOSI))
  (pad 3 smd rect (at 4 0) (size 1 1.8) (layers F.Cu F.Paste F.Mask) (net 9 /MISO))
  (pad 2 smd rect (at 2 0) (size 1 1.8) (layers F.Cu F.Paste F.Mask) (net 7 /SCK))
  (pad 1 smd rect (at 0 0) (size 1 1.8) (layers F.Cu F.Paste F.Mask) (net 20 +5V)))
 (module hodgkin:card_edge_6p (layer F.Cu) (at 88 108)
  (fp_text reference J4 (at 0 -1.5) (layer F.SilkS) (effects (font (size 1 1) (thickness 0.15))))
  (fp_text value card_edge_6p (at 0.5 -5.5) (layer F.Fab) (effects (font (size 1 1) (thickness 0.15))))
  (pad 6 smd rect (at 10 6.1) (size 1 1.8) (layers F.Cu F.Paste F.Mask) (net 57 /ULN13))
  (pad 5 smd rect (at 8 6.1) (size 1 1.8) (layers F.Cu F.Paste F.Mask) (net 13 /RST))
  (pad 4 smd rect (at 6 6.1) (size 1 1.8) (layers F.Cu F.Paste F.Mask) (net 11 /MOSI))
  (pad 3 smd rect (at 4 6.1) (size 1 1.8) (layers F.Cu F.Paste F.Mask) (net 9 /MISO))
  (pad 2 smd rect (at 2 6.1) (size 1 1.8) (layers F.Cu F.Paste F.Mask) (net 7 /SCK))
  (pad 1 smd rect (at 0 6.1) (size 1 1.8) (layers F.Cu F.Paste F.Mask) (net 20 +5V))
  (pad 6 smd rect (at 10 0) (size 1 1.8) (layers F.Cu F.Paste F.Mask) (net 57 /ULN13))
  (pad 5 smd rect (at 8 0) (size 1 1.8) (layers F.Cu F.Paste F.Mask) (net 13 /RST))
  (pad 4 smd rect (at 6 0) (size 1 1.8) (layers F.Cu F.Paste F.Mask) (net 11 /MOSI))
  (pad 3 smd rect (at 4 0) (size 1 1.8) (layers F.Cu F.Paste F.Mask) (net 9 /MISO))
  (pad 2 smd rect (at 2 0) (size 1 1.8) (layers F.Cu F.Paste F.Mask) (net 7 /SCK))
  (pad 1 smd rect (at 0 0) (size 1 1.8) (layers F.Cu F.Paste F.Mask) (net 20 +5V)))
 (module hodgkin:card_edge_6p (layer F.Cu) (at 138 86)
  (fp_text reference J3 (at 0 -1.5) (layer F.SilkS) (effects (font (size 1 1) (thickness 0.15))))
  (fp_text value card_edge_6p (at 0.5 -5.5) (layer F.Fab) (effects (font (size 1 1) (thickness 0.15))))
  (pad 6 smd rect (at 10 6.1) (size 1 1.8) (layers F.Cu F.Paste F.Mask) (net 59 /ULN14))
  (pad 5 smd rect (at 8 6.1) (size 1 1.8) (layers F.Cu F.Paste F.Mask) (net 13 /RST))
  (pad 4 smd rect (at 6 6.1) (size 1 1.8) (layers F.Cu F.Paste F.Mask) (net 11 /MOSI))
  (pad 3 smd rect (at 4 6.1) (size 1 1.8) (layers F.Cu F.Paste F.Mask) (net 9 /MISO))
  (pad 2 smd rect (at 2 6.1) (size 1 1.8) (layers F.Cu F.Paste F.Mask) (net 7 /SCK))
  (pad 1 smd rect (at 0 6.1) (size 1 1.8) (layers F.Cu F.Paste F.Mask) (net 20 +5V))
  (pad 6 smd rect (at 10 0) (size 1 1.8) (layers F.Cu F.Paste F.Mask) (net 59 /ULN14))
  (pad 5 smd rect (at 8 0) (size 1 1.8) (layers F.Cu F.Paste F.Mask) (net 13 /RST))
  (pad 4 smd rect (at 6 0) (size 1 1.8) (layers F.Cu F.Paste F.Mask) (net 11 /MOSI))
  (pad 3 smd rect (at 4 0) (size 1 1.8) (layers F.Cu F.Paste F.Mask) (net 9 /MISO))
  (pad 2 smd rect (at 2 0) (size 1 1.8) (layers F.Cu F.Paste F.Mask) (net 7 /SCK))
  (pad 1 smd rect (at 0 0) (size 1 1.8) (layers F.Cu F.Paste F.Mask) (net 20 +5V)))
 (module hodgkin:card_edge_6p (layer F.Cu) (at 113 86)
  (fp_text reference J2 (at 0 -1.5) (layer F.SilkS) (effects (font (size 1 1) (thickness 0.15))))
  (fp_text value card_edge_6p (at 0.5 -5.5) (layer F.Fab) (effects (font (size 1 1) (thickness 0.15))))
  (pad 6 smd rect (at 10 6.1) (size 1 1.8) (layers F.Cu F.Paste F.Mask) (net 49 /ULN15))
  (pad 5 smd rect (at 8 6.1) (size 1 1.8) (layers F.Cu F.Paste F.Mask) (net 13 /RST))
  (pad 4 smd rect (at 6 6.1) (size 1 1.8) (layers F.Cu F.Paste F.Mask) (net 11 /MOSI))
  (pad 3 smd rect (at 4 6.1) (size 1 1.8) (layers F.Cu F.Paste F.Mask) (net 9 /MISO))
  (pad 2 smd rect (at 2 6.1) (size 1 1.8) (layers F.Cu F.Paste F.Mask) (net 7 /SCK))
  (pad 1 smd rect (at 0 6.1) (size 1 1.8) (layers F.Cu F.Paste F.Mask) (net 20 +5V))
  (pad 6 smd rect (at 10 0) (size 1 1.8) (layers F.Cu F.Paste F.Mask) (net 49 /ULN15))
  (pad 5 smd rect (at 8 0) (size 1 1.8) (layers F.Cu F.Paste F.Mask) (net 13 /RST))
  (pad 4 smd rect (at 6 0) (size 1 1.8) (layers F.Cu F.Paste F.Mask) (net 11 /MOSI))
  (pad 3 smd rect (at 4 0) (size 1 1.8) (layers F.Cu F.Paste F.Mask) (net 9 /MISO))
  (pad 2 smd rect (at 2 0) (size 1 1.8) (layers F.Cu F.Paste F.Mask) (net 7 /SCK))
  (pad 1 smd rect (at 0 0) (size 1 1.8) (layers F.Cu F.Paste F.Mask) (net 20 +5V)))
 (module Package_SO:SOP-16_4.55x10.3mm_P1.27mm (layer B.Cu) (at 117.945 100.25 270)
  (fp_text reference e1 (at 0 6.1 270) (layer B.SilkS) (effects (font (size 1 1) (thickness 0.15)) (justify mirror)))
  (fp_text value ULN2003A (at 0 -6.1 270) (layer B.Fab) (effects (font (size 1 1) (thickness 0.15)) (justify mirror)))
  (pad 16 smd roundrect (at 3.25 4.445 270) (size 1.6 0.6) (layers B.Cu B.Paste B.Mask) (roundrect_rratio 0.25) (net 51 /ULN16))
  (pad 15 smd roundrect (at 3.25 3.175 270) (size 1.6 0.6) (layers B.Cu B.Paste B.Mask) (roundrect_rratio 0.25) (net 49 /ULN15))
  (pad 14 smd roundrect (at 3.25 1.905 270) (size 1.6 0.6) (layers B.Cu B.Paste B.Mask) (roundrect_rratio 0.25) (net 59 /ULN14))
  (pad 13 smd roundrect (at 3.25 0.635 270) (size 1.6 0.6) (layers B.Cu B.Paste B.Mask) (roundrect_rratio 0.25) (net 57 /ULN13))
  (pad 12 smd roundrect (at 3.25 -0.635 270) (size 1.6 0.6) (layers B.Cu B.Paste B.Mask) (roundrect_rratio 0.25) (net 55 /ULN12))
  (pad 11 smd roundrect (at 3.25 -1.905 270) (size 1.6 0.6) (layers B.Cu B.Paste B.Mask) (roundrect_rratio 0.25) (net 53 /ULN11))
  (pad 10 smd roundrect (at 3.25 -3.175 270) (size 1.6 0.6) (layers B.Cu B.Paste B.Mask) (roundrect_rratio 0.25) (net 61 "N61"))
  (pad 9 smd roundrect (at 3.25 -4.445 270) (size 1.6 0.6) (layers B.Cu B.Paste B.Mask) (roundrect_rratio 0.25) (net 20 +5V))
  (pad 8 smd roundrect (at -3.25 -4.445 270) (size 1.6 0.6) (layers B.Cu B.Paste B.Mask) (roundrect_rratio 0.25) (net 5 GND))
  (pad 7 smd roundrect (at -3.25 -3.175 270) (size 1.6 0.6) (layers B.Cu B.Paste B.Mask) (roundrect_rratio 0.25) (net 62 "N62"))
  (pad 6 smd roundrect (at -3.25 -1.905 270) (size 1.6 0.6) (layers B.Cu B.Paste B.Mask) (roundrect_rratio 0.25) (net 25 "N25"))
  (pad 5 smd roundrect (at -3.25 -0.635 270) (size 1.6 0.6) (layers B.Cu B.Paste B.Mask) (roundrect_rratio 0.25) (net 23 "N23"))
  (pad 4 smd roundrect (at -3.25 0.635 270) (size 1.6 0.6) (layers B.Cu B.Paste B.Mask) (roundrect_rratio 0.25) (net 21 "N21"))
  (pad 3 smd roundrect (at -3.25 1.905 270) (size 1.6 0.6) (layers B.Cu B.Paste B.Mask) (roundrect_rratio 0.25) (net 19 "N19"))
  (pad 2 smd roundrect (at -3.25 3.175 270) (size 1.6 0.6) (layers B.Cu B.Paste B.Mask) (roundrect_rratio 0.25) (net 18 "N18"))
  (pad 1 smd roundrect (at -3.25 4.445 270) (size 1.6 0.6) (layers B.Cu B.Paste B.Mask) (roundrect_rratio 0.25) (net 17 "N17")))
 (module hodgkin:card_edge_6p (layer F.Cu) (at 88 86)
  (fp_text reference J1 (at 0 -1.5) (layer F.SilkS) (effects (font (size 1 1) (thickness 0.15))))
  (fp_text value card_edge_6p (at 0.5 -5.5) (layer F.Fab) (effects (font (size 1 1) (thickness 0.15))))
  (pad 6 smd rect (at 10 6.1) (size 1 1.8) (layers F.Cu F.Paste F.Mask) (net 51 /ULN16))
  (pad 5 smd rect (at 8 6.1) (size 1 1.8) (layers F.Cu F.Paste F.Mask) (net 13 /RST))
  (pad 4 smd rect (at 6 6.1) (size 1 1.8) (layers F.Cu F.Paste F.Mask) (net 11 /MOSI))
  (pad 3 smd rect (at 4 6.1) (size 1 1.8) (layers F.Cu F.Paste F.Mask) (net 9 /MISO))
  (pad 2 smd rect (at 2 6.1) (size 1 1.8) (layers F.Cu F.Paste F.Mask) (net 7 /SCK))
  (pad 1 smd rect (at 0 6.1) (size 1 1.8) (layers F.Cu F.Paste F.Mask) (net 20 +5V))
  (pad 6 smd rect (at 10 0) (size 1 1.8) (layers F.Cu F.Paste F.Mask) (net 51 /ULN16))
  (pad 5 smd rect (at 8 0) (size 1 1.8) (layers F.Cu F.Paste F.Mask) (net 13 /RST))
  (pad 4 smd rect (at 6 0) (size 1 1.8) (layers F.Cu F.Paste F.Mask) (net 11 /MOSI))
  (pad 3 smd rect (at 4 0) (size 1 1.8) (layers F.Cu F.Paste F.Mask) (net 9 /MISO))
  (pad 2 smd rect (at 2 0) (size 1 1.8) (layers F.Cu F.Paste F.Mask) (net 7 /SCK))
  (pad 1 smd rect (at 0 0) (size 1 1.8) (layers F.Cu F.Paste F.Mask) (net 20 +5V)))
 (gr_line (start 85 121.7) (end 85 72) (layer Edge.Cuts) (width 0.05))
 (gr_line (start 85 126) (end 85 121.7) (layer Edge.Cuts) (width 0.05))
 (gr_line (start 159.5 126) (end 85 126) (layer Edge.Cuts) (width 0.05))
 (gr_line (start 159.5 72) (end 159.5 126) (layer Edge.Cuts) (width 0.05))
 (gr_line (start 85 72) (end 159.5 72) (layer Edge.Cuts) (width 0.05))
 (segment (start 106.298002 84.775) (end 114.073002 77) (width 0.25) (layer B.Cu) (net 27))
 (segment (start 101.3 84.775) (end 106.298002 84.775) (width 0.25) (layer B.Cu) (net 27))
 (segment (start 142.2 77) (end 144.46 74.74) (width 0.25) (layer B.Cu) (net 27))
 (segment (start 114.073002 77) (end 142.2 77) (width 0.25) (layer B.Cu) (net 27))
 (segment (start 102.3 79.1) (end 101 80.4) (width 0.25) (layer F.Cu) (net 5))
 (segment (start 108.1 79.1) (end 102.3 79.1) (width 0.25) (layer F.Cu) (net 5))
 (segment (start 112.46 74.74) (end 108.1 79.1) (width 0.25) (layer F.Cu) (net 5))
 (via (at 104.1 81.6) (size 0.8) (drill 0.4) (layers F.Cu B.Cu) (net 33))
 (segment (start 102.9 80.4) (end 104.1 81.6) (width 0.25) (layer F.Cu) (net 33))
 (segment (start 102.8 82.9) (end 101.3 82.9) (width 0.25) (layer B.Cu) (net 33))
 (segment (start 104.1 81.6) (end 102.8 82.9) (width 0.25) (layer B.Cu) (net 33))
 (segment (start 101.95 84.8875) (end 103.0625 86) (width 0.25) (layer F.Cu) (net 39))
 (segment (start 101.95 82.4) (end 101.95 84.8875) (width 0.25) (layer F.Cu) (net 39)))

